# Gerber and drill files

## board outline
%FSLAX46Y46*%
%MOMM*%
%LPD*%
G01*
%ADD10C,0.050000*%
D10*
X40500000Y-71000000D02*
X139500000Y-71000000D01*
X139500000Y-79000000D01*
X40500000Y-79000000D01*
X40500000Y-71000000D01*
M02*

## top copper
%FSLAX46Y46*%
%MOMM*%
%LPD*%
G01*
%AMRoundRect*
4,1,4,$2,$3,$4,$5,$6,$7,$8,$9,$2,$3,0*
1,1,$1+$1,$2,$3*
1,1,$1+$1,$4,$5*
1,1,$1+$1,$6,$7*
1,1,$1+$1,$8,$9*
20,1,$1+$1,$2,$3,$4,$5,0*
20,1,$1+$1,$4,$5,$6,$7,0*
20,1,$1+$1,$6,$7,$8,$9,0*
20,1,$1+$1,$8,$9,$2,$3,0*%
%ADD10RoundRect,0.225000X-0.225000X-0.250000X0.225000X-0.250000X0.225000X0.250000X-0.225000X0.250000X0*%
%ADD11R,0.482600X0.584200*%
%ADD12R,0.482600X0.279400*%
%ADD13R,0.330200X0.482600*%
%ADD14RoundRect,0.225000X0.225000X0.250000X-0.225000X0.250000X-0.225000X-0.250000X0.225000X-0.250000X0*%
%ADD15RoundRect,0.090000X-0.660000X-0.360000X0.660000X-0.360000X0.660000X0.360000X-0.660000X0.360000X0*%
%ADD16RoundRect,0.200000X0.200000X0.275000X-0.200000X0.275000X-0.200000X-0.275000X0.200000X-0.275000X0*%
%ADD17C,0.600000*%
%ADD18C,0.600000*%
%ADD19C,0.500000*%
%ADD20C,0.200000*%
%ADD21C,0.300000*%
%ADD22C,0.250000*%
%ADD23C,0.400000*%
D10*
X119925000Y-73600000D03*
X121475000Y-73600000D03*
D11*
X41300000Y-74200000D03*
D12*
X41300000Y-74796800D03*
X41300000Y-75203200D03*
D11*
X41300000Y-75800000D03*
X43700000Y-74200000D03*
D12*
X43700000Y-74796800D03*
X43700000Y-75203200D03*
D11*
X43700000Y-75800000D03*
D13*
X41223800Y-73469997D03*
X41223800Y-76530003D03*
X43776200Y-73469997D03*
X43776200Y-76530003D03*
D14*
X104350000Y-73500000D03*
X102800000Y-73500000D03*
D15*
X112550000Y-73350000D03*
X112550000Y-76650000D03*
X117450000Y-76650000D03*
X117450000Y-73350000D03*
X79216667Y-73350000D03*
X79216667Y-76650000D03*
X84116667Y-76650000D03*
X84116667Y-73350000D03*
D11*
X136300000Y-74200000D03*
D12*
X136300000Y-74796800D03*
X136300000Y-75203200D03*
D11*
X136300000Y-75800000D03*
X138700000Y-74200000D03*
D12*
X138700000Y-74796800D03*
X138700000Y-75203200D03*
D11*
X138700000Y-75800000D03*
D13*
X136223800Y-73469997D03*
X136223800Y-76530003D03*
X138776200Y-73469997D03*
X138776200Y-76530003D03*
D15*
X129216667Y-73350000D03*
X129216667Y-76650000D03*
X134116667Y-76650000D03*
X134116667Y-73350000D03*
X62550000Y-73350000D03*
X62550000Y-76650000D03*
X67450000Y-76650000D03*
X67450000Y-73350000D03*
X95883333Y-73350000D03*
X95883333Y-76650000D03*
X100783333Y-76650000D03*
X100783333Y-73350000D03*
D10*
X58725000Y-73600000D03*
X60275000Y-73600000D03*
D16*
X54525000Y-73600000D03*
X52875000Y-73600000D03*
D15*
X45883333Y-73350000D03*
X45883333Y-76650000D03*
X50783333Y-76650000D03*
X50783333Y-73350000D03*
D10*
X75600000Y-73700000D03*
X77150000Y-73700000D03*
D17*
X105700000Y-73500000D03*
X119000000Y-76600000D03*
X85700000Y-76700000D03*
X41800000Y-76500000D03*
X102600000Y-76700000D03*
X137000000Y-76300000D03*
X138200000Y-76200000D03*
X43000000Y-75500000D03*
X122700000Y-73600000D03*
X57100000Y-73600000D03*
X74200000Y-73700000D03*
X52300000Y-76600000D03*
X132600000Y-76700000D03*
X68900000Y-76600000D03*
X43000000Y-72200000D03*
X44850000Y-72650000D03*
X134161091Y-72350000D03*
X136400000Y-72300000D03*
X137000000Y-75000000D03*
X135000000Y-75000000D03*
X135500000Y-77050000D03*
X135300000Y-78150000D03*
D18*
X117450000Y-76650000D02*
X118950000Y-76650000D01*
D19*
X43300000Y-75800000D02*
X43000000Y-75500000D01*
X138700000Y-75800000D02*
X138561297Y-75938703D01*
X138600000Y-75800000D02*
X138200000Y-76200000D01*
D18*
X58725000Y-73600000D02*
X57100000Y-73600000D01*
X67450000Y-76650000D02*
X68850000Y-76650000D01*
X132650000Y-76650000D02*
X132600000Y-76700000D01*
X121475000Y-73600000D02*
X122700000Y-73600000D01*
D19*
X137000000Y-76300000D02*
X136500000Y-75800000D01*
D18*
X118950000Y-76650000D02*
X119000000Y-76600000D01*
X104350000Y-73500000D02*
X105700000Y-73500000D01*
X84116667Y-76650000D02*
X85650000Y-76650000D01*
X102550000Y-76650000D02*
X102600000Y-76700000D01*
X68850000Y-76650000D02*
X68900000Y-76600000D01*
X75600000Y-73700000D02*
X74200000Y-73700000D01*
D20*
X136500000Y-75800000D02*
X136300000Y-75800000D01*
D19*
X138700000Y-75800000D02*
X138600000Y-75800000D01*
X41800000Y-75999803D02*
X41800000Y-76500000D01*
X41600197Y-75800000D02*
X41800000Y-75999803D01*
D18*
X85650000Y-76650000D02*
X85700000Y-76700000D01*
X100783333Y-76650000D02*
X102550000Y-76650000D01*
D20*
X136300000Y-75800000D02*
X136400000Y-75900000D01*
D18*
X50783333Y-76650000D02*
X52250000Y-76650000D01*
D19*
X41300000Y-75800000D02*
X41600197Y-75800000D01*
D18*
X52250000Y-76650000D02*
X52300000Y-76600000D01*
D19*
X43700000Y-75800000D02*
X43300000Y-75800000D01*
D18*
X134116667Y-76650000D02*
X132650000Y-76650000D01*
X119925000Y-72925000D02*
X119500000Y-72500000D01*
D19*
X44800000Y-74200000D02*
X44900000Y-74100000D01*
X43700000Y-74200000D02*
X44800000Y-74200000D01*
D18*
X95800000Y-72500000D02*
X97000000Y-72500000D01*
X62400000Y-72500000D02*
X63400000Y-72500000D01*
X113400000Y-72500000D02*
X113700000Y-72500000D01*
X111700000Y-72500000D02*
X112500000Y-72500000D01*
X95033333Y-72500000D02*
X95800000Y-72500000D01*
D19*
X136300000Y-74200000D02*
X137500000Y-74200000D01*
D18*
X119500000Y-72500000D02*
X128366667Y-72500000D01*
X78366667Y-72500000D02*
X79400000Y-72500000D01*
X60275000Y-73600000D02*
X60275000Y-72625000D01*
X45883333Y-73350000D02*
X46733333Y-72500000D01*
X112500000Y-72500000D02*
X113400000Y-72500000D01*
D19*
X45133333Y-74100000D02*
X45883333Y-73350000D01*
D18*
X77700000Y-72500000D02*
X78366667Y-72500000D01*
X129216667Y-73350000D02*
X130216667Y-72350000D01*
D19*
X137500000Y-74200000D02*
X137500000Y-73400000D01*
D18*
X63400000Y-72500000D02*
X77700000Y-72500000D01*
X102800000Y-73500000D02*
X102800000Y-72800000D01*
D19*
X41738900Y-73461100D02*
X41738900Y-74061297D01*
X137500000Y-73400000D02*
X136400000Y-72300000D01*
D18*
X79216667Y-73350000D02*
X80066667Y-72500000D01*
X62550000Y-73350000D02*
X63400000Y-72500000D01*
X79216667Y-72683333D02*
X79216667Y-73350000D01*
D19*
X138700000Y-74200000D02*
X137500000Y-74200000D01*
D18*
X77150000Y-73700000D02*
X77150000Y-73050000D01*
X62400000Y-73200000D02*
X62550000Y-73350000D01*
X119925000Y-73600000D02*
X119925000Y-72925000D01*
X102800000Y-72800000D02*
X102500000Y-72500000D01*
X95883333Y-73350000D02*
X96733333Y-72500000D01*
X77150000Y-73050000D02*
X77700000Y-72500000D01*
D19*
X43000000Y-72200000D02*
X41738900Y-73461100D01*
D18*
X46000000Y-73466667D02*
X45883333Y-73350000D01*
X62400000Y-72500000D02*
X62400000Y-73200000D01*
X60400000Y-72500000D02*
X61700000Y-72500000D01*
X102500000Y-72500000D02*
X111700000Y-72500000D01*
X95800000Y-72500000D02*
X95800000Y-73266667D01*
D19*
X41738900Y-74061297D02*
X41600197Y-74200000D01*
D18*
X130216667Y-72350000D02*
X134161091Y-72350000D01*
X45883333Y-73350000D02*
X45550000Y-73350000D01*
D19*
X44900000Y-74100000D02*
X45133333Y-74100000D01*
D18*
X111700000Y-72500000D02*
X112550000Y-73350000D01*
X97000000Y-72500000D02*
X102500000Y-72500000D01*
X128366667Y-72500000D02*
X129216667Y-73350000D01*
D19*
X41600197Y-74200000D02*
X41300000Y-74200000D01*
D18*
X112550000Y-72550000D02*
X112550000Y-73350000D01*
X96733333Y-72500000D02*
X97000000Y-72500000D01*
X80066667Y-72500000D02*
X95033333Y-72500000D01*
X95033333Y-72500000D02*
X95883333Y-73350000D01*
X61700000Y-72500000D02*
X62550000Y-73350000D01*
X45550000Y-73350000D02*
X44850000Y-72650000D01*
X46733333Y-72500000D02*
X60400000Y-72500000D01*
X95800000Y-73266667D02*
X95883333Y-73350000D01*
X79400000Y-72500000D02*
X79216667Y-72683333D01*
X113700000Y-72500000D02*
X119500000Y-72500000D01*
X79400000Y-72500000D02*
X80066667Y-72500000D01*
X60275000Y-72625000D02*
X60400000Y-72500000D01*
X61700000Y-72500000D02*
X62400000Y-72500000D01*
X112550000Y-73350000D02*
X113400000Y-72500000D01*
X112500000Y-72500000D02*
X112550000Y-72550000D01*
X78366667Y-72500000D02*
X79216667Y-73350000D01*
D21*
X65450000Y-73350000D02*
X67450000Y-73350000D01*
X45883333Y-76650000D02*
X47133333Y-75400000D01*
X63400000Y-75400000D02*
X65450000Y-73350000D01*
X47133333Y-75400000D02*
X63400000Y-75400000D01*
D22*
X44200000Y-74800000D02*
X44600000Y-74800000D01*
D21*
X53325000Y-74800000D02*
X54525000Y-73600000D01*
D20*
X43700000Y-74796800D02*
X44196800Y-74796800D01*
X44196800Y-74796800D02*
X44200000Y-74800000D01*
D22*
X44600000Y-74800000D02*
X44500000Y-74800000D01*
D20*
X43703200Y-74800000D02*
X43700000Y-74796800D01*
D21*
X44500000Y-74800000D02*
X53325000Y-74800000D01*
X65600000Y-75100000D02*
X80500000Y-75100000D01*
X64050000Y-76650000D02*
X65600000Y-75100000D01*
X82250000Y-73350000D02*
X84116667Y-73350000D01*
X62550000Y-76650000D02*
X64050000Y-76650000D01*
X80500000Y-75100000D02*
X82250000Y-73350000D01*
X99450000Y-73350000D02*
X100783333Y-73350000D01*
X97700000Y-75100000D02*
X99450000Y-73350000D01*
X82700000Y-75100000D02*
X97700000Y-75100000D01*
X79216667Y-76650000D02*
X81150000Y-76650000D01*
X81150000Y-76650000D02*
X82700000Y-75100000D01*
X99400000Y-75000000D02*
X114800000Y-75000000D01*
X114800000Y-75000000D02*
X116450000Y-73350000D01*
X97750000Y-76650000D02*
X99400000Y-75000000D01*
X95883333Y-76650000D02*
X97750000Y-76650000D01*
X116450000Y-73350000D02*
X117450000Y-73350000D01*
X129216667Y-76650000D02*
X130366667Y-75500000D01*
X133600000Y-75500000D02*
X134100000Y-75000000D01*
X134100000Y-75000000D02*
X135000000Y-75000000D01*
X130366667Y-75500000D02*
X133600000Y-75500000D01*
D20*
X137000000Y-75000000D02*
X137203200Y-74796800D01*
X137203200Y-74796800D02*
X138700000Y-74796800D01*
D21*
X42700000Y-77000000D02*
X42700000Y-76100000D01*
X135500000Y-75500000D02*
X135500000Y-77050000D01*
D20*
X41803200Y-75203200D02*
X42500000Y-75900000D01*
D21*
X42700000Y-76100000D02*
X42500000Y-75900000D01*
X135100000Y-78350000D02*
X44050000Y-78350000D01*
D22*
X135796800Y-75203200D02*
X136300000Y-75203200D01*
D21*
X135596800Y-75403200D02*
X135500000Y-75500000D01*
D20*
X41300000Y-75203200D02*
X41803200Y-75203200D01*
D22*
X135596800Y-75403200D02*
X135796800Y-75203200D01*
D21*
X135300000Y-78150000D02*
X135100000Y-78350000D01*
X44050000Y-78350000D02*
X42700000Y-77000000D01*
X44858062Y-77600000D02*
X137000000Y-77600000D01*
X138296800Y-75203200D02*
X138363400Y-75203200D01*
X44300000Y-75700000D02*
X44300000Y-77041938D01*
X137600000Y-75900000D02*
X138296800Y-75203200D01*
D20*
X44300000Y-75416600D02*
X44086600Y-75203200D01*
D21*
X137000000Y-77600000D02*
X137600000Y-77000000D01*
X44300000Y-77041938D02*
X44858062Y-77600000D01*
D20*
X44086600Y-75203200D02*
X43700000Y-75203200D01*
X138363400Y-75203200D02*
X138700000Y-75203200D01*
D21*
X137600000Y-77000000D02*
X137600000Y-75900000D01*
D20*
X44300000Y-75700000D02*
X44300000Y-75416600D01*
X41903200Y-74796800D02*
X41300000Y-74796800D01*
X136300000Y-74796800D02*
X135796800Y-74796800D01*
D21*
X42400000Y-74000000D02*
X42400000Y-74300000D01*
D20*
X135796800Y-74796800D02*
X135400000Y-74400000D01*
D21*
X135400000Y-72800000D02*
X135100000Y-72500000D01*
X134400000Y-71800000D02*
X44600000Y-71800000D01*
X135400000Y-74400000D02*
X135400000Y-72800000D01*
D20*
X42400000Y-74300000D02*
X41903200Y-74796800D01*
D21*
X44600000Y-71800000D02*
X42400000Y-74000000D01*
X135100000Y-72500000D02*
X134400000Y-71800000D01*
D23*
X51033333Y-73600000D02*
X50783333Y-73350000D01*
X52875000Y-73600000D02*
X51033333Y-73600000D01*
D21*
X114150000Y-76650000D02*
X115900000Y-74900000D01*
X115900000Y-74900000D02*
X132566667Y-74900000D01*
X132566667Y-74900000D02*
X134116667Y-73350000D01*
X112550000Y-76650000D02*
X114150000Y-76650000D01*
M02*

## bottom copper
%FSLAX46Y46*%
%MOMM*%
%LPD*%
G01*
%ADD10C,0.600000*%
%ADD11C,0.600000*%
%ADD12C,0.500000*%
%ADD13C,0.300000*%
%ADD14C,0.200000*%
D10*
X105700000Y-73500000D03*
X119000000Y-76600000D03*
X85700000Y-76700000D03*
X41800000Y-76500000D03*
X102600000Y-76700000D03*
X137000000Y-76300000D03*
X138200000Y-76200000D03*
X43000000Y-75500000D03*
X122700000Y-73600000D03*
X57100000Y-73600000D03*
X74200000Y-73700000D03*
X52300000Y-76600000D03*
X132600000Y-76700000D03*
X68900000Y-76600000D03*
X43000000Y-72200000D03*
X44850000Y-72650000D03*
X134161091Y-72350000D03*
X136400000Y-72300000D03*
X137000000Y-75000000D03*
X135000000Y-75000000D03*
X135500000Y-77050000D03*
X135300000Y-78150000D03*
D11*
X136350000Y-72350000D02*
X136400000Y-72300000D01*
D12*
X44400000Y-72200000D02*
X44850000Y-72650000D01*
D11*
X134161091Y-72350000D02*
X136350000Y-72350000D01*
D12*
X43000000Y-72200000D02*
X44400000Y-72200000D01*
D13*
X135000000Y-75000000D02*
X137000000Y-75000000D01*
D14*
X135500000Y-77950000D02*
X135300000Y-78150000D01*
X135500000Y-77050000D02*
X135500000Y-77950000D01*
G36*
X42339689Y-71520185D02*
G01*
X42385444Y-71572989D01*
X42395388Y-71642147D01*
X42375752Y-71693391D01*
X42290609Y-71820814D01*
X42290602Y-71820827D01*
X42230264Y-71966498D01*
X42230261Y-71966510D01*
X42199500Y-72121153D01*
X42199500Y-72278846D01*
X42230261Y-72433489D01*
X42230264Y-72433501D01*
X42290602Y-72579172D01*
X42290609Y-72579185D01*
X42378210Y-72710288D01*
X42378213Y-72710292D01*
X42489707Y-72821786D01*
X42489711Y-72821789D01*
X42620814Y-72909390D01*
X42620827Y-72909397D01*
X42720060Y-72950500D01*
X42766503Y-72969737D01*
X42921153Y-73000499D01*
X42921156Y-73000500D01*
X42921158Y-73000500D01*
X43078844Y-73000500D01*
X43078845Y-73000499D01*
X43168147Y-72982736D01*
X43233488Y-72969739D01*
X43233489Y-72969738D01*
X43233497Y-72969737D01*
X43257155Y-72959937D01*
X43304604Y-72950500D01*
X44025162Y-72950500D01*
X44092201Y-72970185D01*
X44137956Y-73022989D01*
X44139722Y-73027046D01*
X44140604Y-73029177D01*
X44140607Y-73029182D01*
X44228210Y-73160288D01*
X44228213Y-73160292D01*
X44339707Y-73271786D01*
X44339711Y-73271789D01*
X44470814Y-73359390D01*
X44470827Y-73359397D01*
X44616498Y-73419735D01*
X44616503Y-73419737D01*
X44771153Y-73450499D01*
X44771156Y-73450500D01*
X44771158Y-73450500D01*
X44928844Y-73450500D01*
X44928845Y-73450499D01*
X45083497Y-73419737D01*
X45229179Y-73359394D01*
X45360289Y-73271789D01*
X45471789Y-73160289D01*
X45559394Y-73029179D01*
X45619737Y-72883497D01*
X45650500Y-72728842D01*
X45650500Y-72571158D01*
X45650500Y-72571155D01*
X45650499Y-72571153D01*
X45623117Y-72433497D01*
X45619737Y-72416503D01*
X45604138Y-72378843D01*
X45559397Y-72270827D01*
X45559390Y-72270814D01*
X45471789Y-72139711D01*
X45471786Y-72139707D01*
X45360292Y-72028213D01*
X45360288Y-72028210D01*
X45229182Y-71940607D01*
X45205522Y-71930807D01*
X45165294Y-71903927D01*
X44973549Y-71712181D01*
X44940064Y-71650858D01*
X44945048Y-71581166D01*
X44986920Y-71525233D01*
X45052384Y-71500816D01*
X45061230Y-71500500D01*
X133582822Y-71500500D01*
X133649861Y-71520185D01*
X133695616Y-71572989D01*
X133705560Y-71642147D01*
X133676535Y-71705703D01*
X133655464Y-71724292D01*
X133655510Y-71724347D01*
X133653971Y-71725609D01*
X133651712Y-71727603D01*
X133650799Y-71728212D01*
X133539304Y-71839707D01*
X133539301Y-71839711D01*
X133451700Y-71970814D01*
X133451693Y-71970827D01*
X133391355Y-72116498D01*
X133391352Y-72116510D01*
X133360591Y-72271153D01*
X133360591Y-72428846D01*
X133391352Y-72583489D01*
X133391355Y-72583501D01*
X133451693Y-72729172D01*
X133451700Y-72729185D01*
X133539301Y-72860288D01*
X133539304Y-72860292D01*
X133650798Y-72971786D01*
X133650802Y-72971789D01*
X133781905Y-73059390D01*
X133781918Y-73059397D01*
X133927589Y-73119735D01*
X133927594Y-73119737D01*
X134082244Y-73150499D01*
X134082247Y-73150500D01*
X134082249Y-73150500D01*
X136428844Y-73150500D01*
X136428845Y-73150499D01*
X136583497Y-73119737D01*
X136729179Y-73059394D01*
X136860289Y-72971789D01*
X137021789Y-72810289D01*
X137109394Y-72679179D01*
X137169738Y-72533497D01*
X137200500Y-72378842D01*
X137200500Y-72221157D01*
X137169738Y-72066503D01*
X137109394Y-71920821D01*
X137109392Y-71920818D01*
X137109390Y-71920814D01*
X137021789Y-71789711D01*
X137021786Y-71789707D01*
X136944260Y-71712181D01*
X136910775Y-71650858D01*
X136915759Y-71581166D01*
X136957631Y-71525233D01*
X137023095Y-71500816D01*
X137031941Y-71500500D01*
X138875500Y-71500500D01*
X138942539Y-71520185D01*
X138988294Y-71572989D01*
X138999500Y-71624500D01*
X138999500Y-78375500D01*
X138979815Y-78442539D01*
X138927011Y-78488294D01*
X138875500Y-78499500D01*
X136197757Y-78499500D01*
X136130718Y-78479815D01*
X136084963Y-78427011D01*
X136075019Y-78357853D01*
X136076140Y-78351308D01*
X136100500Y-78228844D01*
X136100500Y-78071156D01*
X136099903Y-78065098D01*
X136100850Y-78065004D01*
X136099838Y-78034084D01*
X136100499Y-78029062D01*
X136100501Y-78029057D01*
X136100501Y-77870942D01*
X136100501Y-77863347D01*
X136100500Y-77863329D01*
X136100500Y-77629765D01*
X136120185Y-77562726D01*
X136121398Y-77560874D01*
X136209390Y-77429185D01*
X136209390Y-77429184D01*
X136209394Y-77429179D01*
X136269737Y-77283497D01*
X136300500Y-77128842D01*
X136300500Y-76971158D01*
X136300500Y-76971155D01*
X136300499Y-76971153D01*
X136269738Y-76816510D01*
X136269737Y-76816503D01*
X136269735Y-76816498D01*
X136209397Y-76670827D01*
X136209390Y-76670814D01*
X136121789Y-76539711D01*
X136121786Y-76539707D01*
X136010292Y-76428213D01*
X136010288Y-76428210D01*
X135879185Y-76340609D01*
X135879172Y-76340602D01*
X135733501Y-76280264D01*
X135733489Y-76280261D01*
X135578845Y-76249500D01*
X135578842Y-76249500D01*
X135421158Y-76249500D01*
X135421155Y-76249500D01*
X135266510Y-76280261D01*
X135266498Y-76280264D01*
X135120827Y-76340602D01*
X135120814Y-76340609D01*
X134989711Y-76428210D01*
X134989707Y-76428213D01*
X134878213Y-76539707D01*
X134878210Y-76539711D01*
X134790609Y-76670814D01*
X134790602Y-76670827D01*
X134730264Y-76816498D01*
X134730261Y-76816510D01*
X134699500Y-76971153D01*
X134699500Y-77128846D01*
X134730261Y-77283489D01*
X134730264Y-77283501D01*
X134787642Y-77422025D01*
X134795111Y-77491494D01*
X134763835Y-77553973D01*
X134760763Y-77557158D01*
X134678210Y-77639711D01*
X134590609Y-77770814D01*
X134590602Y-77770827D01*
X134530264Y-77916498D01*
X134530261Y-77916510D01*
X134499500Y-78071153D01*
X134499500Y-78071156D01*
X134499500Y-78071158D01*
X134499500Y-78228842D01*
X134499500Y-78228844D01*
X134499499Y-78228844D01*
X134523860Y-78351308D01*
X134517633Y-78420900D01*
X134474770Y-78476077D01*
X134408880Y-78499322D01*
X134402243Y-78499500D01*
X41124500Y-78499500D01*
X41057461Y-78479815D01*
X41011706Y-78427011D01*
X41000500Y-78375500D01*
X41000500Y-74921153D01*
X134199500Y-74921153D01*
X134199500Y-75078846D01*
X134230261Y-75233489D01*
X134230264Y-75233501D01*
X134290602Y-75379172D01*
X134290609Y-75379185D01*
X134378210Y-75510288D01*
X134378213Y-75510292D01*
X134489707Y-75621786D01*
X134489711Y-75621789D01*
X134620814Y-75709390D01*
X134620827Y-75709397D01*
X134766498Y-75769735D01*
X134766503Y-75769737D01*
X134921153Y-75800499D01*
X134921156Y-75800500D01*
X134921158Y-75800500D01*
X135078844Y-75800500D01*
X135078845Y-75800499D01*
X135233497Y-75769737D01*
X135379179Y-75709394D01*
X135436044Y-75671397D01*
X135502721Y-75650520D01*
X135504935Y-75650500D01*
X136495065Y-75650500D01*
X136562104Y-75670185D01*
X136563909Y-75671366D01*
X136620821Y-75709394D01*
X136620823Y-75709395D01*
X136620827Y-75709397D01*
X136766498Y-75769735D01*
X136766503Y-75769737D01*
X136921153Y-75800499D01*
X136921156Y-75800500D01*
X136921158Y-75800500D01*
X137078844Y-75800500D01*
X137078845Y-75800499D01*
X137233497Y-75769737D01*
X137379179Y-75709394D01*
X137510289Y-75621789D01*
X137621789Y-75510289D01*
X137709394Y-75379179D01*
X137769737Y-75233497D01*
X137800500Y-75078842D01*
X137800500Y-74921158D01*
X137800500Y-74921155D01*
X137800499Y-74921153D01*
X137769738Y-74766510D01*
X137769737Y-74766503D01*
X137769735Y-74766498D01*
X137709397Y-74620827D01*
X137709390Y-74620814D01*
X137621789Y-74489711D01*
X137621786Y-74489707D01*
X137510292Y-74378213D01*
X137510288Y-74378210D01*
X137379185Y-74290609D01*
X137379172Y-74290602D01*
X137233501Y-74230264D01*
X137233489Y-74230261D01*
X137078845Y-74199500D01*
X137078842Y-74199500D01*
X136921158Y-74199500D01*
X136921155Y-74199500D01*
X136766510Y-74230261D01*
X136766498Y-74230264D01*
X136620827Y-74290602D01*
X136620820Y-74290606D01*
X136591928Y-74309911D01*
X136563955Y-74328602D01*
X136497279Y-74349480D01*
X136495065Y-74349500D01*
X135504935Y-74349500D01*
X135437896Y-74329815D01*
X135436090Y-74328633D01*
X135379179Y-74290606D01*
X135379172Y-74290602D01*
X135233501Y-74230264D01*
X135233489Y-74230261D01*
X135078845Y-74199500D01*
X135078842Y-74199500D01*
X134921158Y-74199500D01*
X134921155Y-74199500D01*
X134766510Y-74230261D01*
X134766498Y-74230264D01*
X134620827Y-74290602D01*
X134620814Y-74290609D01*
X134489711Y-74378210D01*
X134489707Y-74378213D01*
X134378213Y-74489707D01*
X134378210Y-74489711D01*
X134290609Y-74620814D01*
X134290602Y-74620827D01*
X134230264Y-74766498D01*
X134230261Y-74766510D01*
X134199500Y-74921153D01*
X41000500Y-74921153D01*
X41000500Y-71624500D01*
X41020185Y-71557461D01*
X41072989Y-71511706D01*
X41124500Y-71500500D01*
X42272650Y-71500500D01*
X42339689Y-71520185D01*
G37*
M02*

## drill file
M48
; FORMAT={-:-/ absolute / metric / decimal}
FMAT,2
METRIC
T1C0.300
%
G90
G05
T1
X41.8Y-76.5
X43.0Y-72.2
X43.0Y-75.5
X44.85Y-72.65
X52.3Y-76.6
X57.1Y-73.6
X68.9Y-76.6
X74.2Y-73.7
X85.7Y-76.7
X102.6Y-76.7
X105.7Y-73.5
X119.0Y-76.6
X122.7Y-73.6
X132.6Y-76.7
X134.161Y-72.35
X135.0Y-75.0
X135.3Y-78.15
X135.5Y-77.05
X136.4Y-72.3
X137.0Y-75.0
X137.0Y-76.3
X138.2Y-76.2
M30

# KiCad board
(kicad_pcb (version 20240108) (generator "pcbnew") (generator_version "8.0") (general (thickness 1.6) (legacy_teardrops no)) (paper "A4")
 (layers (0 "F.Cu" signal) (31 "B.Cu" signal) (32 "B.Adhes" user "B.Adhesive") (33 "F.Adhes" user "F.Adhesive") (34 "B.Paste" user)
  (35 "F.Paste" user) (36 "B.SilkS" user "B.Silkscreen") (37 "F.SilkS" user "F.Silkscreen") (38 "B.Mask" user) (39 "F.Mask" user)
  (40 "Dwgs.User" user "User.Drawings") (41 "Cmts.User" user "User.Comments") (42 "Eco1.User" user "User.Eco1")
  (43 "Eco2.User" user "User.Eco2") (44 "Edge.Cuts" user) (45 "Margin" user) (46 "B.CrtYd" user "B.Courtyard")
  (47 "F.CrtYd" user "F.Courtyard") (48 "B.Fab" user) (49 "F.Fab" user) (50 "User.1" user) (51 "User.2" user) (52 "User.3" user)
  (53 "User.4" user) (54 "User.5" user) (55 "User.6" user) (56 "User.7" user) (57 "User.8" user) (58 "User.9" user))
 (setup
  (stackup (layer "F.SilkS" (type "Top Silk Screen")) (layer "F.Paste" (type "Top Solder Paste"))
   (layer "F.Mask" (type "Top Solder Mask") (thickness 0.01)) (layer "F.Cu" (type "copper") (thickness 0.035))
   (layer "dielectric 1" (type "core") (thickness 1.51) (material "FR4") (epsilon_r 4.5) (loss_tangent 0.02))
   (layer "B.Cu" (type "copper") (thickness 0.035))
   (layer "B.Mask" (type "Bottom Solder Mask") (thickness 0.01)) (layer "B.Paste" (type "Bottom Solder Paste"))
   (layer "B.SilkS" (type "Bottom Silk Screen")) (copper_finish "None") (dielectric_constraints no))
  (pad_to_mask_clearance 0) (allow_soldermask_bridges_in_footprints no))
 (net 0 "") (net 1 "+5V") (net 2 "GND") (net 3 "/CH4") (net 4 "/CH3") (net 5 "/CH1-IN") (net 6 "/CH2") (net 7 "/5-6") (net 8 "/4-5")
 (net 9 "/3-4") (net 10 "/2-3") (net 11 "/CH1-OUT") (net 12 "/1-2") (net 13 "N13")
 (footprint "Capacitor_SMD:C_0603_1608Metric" (layer "F.Cu") (at 120.7 73.6)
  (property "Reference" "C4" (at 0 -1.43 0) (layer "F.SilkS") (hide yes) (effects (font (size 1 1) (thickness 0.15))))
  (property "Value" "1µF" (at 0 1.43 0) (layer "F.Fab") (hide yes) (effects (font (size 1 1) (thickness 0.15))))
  (pad "1" smd roundrect (at -0.775 0) (size 0.9 0.95) (layers "F.Cu" "F.Paste" "F.Mask") (roundrect_rratio 0.25) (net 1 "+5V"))
  (pad "2" smd roundrect (at 0.775 0) (size 0.9 0.95) (layers "F.Cu" "F.Paste" "F.Mask") (roundrect_rratio 0.25) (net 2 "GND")))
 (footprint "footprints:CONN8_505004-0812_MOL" (layer "F.Cu") (at 42.5 75 90)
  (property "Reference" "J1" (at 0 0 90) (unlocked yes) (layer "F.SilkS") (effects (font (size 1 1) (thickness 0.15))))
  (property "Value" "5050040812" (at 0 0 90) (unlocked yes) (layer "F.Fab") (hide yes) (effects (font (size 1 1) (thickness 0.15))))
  (pad "1" smd rect (at 0.8 -1.2 90) (size 0.5842 0.4826) (layers "F.Cu" "F.Paste" "F.Mask") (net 1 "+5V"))
  (pad "2" smd rect (at 0.2032 -1.2 90) (size 0.2794 0.4826) (layers "F.Cu" "F.Paste" "F.Mask") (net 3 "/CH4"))
  (pad "3" smd rect (at -0.2032 -1.2 90) (size 0.2794 0.4826) (layers "F.Cu" "F.Paste" "F.Mask") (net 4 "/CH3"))
  (pad "4" smd rect (at -0.8 -1.2 90) (size 0.5842 0.4826) (layers "F.Cu" "F.Paste" "F.Mask") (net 2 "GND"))
  (pad "5" smd rect (at 0.8 1.2 90) (size 0.5842 0.4826) (layers "F.Cu" "F.Paste" "F.Mask") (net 1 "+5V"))
  (pad "6" smd rect (at 0.2032 1.2 90) (size 0.2794 0.4826) (layers "F.Cu" "F.Paste" "F.Mask") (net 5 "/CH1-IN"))
  (pad "7" smd rect (at -0.2032 1.2 90) (size 0.2794 0.4826) (layers "F.Cu" "F.Paste" "F.Mask") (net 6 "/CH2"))
  (pad "8" smd rect (at -0.8 1.2 90) (size 0.5842 0.4826) (layers "F.Cu" "F.Paste" "F.Mask") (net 2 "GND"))
  (pad "9" smd rect (at 1.530003 -1.2762 90) (size 0.4826 0.3302) (layers "F.Cu" "F.Paste" "F.Mask"))
  (pad "10" smd rect (at -1.530003 -1.2762 90) (size 0.4826 0.3302) (layers "F.Cu" "F.Paste" "F.Mask"))
  (pad "11" smd rect (at 1.530003 1.2762 90) (size 0.4826 0.3302) (layers "F.Cu" "F.Paste" "F.Mask"))
  (pad "12" smd rect (at -1.530003 1.2762 90) (size 0.4826 0.3302) (layers "F.Cu" "F.Paste" "F.Mask")))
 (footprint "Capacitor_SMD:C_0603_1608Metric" (layer "F.Cu") (at 103.575 73.5 180)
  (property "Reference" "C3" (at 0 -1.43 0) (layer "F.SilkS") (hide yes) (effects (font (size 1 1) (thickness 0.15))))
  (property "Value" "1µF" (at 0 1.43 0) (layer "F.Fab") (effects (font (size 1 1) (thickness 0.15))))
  (pad "1" smd roundrect (at -0.775 0 180) (size 0.9 0.95) (layers "F.Cu" "F.Paste" "F.Mask") (roundrect_rratio 0.25) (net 2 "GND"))
  (pad "2" smd roundrect (at 0.775 0 180) (size 0.9 0.95) (layers "F.Cu" "F.Paste" "F.Mask") (roundrect_rratio 0.25) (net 1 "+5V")))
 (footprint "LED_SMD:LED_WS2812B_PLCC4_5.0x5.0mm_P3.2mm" (layer "F.Cu") (at 115 75)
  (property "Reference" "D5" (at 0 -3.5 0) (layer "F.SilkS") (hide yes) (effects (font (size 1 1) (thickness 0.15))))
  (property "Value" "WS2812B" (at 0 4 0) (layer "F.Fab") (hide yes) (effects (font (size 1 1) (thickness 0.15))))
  (pad "1" smd roundrect (at -2.45 -1.65) (size 1.5 0.9) (layers "F.Cu" "F.Paste" "F.Mask") (roundrect_rratio 0.1) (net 1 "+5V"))
  (pad "2" smd roundrect (at -2.45 1.65) (size 1.5 0.9) (layers "F.Cu" "F.Paste" "F.Mask") (roundrect_rratio 0.1) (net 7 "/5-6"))
  (pad "3" smd roundrect (at 2.45 1.65) (size 1.5 0.9) (layers "F.Cu" "F.Paste" "F.Mask") (roundrect_rratio 0.1) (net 2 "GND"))
  (pad "4" smd roundrect (at 2.45 -1.65) (size 1.5 0.9) (layers "F.Cu" "F.Paste" "F.Mask") (roundrect_rratio 0.1) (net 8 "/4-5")))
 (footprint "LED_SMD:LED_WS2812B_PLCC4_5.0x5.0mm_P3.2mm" (layer "F.Cu") (at 81.666667 75)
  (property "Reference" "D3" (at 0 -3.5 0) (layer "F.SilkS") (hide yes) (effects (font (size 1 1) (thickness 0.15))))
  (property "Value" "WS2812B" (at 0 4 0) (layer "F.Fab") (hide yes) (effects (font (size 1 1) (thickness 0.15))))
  (pad "1" smd roundrect (at -2.45 -1.65) (size 1.5 0.9) (layers "F.Cu" "F.Paste" "F.Mask") (roundrect_rratio 0.1) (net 1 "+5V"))
  (pad "2" smd roundrect (at -2.45 1.65) (size 1.5 0.9) (layers "F.Cu" "F.Paste" "F.Mask") (roundrect_rratio 0.1) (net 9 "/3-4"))
  (pad "3" smd roundrect (at 2.45 1.65) (size 1.5 0.9) (layers "F.Cu" "F.Paste" "F.Mask") (roundrect_rratio 0.1) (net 2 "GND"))
  (pad "4" smd roundrect (at 2.45 -1.65) (size 1.5 0.9) (layers "F.Cu" "F.Paste" "F.Mask") (roundrect_rratio 0.1) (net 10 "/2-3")))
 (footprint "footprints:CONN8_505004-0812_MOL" (layer "F.Cu") (at 137.5 75 90)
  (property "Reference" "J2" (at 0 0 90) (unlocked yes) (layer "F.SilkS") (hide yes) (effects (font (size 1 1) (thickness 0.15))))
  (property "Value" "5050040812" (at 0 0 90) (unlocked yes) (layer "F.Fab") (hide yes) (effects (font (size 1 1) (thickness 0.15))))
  (pad "1" smd rect (at 0.8 -1.2 90) (size 0.5842 0.4826) (layers "F.Cu" "F.Paste" "F.Mask") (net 1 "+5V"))
  (pad "2" smd rect (at 0.2032 -1.2 90) (size 0.2794 0.4826) (layers "F.Cu" "F.Paste" "F.Mask") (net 3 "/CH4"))
  (pad "3" smd rect (at -0.2032 -1.2 90) (size 0.2794 0.4826) (layers "F.Cu" "F.Paste" "F.Mask") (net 4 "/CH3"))
  (pad "4" smd rect (at -0.8 -1.2 90) (size 0.5842 0.4826) (layers "F.Cu" "F.Paste" "F.Mask") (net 2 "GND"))
  (pad "5" smd rect (at 0.8 1.2 90) (size 0.5842 0.4826) (layers "F.Cu" "F.Paste" "F.Mask") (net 1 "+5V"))
  (pad "6" smd rect (at 0.2032 1.2 90) (size 0.2794 0.4826) (layers "F.Cu" "F.Paste" "F.Mask") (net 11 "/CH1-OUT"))
  (pad "7" smd rect (at -0.2032 1.2 90) (size 0.2794 0.4826) (layers "F.Cu" "F.Paste" "F.Mask") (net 6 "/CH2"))
  (pad "8" smd rect (at -0.8 1.2 90) (size 0.5842 0.4826) (layers "F.Cu" "F.Paste" "F.Mask") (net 2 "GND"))
  (pad "9" smd rect (at 1.530003 -1.2762 90) (size 0.4826 0.3302) (layers "F.Cu" "F.Paste" "F.Mask"))
  (pad "10" smd rect (at -1.530003 -1.2762 90) (size 0.4826 0.3302) (layers "F.Cu" "F.Paste" "F.Mask"))
  (pad "11" smd rect (at 1.530003 1.2762 90) (size 0.4826 0.3302) (layers "F.Cu" "F.Paste" "F.Mask"))
  (pad "12" smd rect (at -1.530003 1.2762 90) (size 0.4826 0.3302) (layers "F.Cu" "F.Paste" "F.Mask")))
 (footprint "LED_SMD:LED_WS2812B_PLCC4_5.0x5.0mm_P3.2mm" (layer "F.Cu") (at 131.666667 75)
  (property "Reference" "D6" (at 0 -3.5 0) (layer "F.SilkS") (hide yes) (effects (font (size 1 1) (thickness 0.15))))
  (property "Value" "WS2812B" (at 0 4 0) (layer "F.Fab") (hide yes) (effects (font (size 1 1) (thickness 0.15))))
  (pad "1" smd roundrect (at -2.45 -1.65) (size 1.5 0.9) (layers "F.Cu" "F.Paste" "F.Mask") (roundrect_rratio 0.1) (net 1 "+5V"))
  (pad "2" smd roundrect (at -2.45 1.65) (size 1.5 0.9) (layers "F.Cu" "F.Paste" "F.Mask") (roundrect_rratio 0.1) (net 11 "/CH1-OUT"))
  (pad "3" smd roundrect (at 2.45 1.65) (size 1.5 0.9) (layers "F.Cu" "F.Paste" "F.Mask") (roundrect_rratio 0.1) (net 2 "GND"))
  (pad "4" smd roundrect (at 2.45 -1.65) (size 1.5 0.9) (layers "F.Cu" "F.Paste" "F.Mask") (roundrect_rratio 0.1) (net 7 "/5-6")))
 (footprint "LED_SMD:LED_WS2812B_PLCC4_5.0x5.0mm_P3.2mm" (layer "F.Cu") (at 65 75)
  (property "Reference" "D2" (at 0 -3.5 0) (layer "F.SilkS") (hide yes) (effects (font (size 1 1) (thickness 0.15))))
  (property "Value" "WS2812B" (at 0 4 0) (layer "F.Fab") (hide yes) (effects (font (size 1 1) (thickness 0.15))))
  (pad "1" smd roundrect (at -2.45 -1.65) (size 1.5 0.9) (layers "F.Cu" "F.Paste" "F.Mask") (roundrect_rratio 0.1) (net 1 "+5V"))
  (pad "2" smd roundrect (at -2.45 1.65) (size 1.5 0.9) (layers "F.Cu" "F.Paste" "F.Mask") (roundrect_rratio 0.1) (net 10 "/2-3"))
  (pad "3" smd roundrect (at 2.45 1.65) (size 1.5 0.9) (layers "F.Cu" "F.Paste" "F.Mask") (roundrect_rratio 0.1) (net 2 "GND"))
  (pad "4" smd roundrect (at 2.45 -1.65) (size 1.5 0.9) (layers "F.Cu" "F.Paste" "F.Mask") (roundrect_rratio 0.1) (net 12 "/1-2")))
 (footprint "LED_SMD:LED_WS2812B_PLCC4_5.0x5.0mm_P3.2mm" (layer "F.Cu") (at 98.333333 75)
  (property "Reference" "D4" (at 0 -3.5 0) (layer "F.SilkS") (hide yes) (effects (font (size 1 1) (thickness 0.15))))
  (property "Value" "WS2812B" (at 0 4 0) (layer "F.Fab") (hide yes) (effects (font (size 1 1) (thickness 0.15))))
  (pad "1" smd roundrect (at -2.45 -1.65) (size 1.5 0.9) (layers "F.Cu" "F.Paste" "F.Mask") (roundrect_rratio 0.1) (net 1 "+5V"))
  (pad "2" smd roundrect (at -2.45 1.65) (size 1.5 0.9) (layers "F.Cu" "F.Paste" "F.Mask") (roundrect_rratio 0.1) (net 8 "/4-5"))
  (pad "3" smd roundrect (at 2.45 1.65) (size 1.5 0.9) (layers "F.Cu" "F.Paste" "F.Mask") (roundrect_rratio 0.1) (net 2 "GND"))
  (pad "4" smd roundrect (at 2.45 -1.65) (size 1.5 0.9) (layers "F.Cu" "F.Paste" "F.Mask") (roundrect_rratio 0.1) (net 9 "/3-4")))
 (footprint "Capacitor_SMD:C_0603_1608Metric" (layer "F.Cu") (at 59.5 73.6)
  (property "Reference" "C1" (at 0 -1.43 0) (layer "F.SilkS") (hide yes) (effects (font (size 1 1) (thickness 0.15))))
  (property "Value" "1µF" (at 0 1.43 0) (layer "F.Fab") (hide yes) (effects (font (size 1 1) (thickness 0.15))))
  (pad "1" smd roundrect (at -0.775 0) (size 0.9 0.95) (layers "F.Cu" "F.Paste" "F.Mask") (roundrect_rratio 0.25) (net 2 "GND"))
  (pad "2" smd roundrect (at 0.775 0) (size 0.9 0.95) (layers "F.Cu" "F.Paste" "F.Mask") (roundrect_rratio 0.25) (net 1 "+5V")))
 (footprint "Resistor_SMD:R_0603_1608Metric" (layer "F.Cu") (at 53.7 73.6 180)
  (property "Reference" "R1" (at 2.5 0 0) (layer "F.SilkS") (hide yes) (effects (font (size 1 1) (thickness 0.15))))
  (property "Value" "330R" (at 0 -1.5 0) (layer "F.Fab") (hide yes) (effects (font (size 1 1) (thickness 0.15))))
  (pad "1" smd roundrect (at -0.825 0 180) (size 0.8 0.95) (layers "F.Cu" "F.Paste" "F.Mask") (roundrect_rratio 0.25) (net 5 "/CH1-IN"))
  (pad "2" smd roundrect (at 0.825 0 180) (size 0.8 0.95) (layers "F.Cu" "F.Paste" "F.Mask") (roundrect_rratio 0.25) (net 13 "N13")))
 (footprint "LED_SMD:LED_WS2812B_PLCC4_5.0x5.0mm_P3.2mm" (layer "F.Cu") (at 48.333333 75)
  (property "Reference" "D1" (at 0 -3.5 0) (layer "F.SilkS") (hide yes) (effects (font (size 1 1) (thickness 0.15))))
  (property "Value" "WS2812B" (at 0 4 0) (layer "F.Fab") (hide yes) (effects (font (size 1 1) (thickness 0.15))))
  (pad "1" smd roundrect (at -2.45 -1.65) (size 1.5 0.9) (layers "F.Cu" "F.Paste" "F.Mask") (roundrect_rratio 0.1) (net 1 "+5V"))
  (pad "2" smd roundrect (at -2.45 1.65) (size 1.5 0.9) (layers "F.Cu" "F.Paste" "F.Mask") (roundrect_rratio 0.1) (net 12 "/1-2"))
  (pad "3" smd roundrect (at 2.45 1.65) (size 1.5 0.9) (layers "F.Cu" "F.Paste" "F.Mask") (roundrect_rratio 0.1) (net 2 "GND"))
  (pad "4" smd roundrect (at 2.45 -1.65) (size 1.5 0.9) (layers "F.Cu" "F.Paste" "F.Mask") (roundrect_rratio 0.1) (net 13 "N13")))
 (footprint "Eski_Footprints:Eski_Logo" (layer "F.Cu") (at 90 76.85)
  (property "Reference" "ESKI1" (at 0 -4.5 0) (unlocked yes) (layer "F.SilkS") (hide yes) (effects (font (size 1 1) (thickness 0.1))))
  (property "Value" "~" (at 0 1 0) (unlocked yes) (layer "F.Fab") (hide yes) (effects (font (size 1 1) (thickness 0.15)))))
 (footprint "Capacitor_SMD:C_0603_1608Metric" (layer "F.Cu") (at 76.375 73.7)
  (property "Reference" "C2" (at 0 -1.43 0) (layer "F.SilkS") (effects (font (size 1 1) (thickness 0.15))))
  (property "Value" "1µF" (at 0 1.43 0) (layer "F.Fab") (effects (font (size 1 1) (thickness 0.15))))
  (pad "1" smd roundrect (at -0.775 0) (size 0.9 0.95) (layers "F.Cu" "F.Paste" "F.Mask") (roundrect_rratio 0.25) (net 2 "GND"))
  (pad "2" smd roundrect (at 0.775 0) (size 0.9 0.95) (layers "F.Cu" "F.Paste" "F.Mask") (roundrect_rratio 0.25) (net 1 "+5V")))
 (gr_rect (start 40.5 71) (end 139.5 79) (stroke (width 0.05) (type default)) (fill none) (layer "Edge.Cuts"))
 (segment (start 117.45 76.65) (end 118.95 76.65) (width 0.6) (layer "F.Cu") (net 2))
 (segment (start 43.3 75.8) (end 43 75.5) (width 0.5) (layer "F.Cu") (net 2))
 (segment (start 138.7 75.8) (end 138.561297 75.938703) (width 0.5) (layer "F.Cu") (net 2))
 (segment (start 138.6 75.8) (end 138.2 76.2) (width 0.5) (layer "F.Cu") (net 2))
 (segment (start 58.725 73.6) (end 57.1 73.6) (width 0.6) (layer "F.Cu") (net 2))
 (segment (start 67.45 76.65) (end 68.85 76.65) (width 0.6) (layer "F.Cu") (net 2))
 (segment (start 132.65 76.65) (end 132.6 76.7) (width 0.6) (layer "F.Cu") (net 2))
 (segment (start 121.475 73.6) (end 122.7 73.6) (width 0.6) (layer "F.Cu") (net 2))
 (segment (start 137 76.3) (end 136.5 75.8) (width 0.5) (layer "F.Cu") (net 2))
 (segment (start 118.95 76.65) (end 119 76.6) (width 0.6) (layer "F.Cu") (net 2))
 (segment (start 104.35 73.5) (end 105.7 73.5) (width 0.6) (layer "F.Cu") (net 2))
 (segment (start 84.116667 76.65) (end 85.65 76.65) (width 0.6) (layer "F.Cu") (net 2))
 (segment (start 102.55 76.65) (end 102.6 76.7) (width 0.6) (layer "F.Cu") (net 2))
 (segment (start 68.85 76.65) (end 68.9 76.6) (width 0.6) (layer "F.Cu") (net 2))
 (segment (start 75.6 73.7) (end 74.2 73.7) (width 0.6) (layer "F.Cu") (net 2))
 (segment (start 136.5 75.8) (end 136.3 75.8) (width 0.2) (layer "F.Cu") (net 2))
 (segment (start 138.7 75.8) (end 138.6 75.8) (width 0.5) (layer "F.Cu") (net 2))
 (segment (start 41.8 75.999803) (end 41.8 76.5) (width 0.5) (layer "F.Cu") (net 2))
 (segment (start 41.600197 75.8) (end 41.8 75.999803) (width 0.5) (layer "F.Cu") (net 2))
 (segment (start 85.65 76.65) (end 85.7 76.7) (width 0.6) (layer "F.Cu") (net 2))
 (segment (start 100.783333 76.65) (end 102.55 76.65) (width 0.6) (layer "F.Cu") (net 2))
 (segment (start 136.3 75.8) (end 136.4 75.9) (width 0.2) (layer "F.Cu") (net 2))
 (segment (start 50.783333 76.65) (end 52.25 76.65) (width 0.6) (layer "F.Cu") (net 2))
 (segment (start 41.3 75.8) (end 41.600197 75.8) (width 0.5) (layer "F.Cu") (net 2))
 (segment (start 52.25 76.65) (end 52.3 76.6) (width 0.6) (layer "F.Cu") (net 2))
 (segment (start 43.7 75.8) (end 43.3 75.8) (width 0.5) (layer "F.Cu") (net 2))
 (segment (start 134.116667 76.65) (end 132.65 76.65) (width 0.6) (layer "F.Cu") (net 2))
 (via (at 105.7 73.5) (size 0.6) (drill 0.3) (layers "F.Cu" "B.Cu") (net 2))
 (via (at 119 76.6) (size 0.6) (drill 0.3) (layers "F.Cu" "B.Cu") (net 2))
 (via (at 85.7 76.7) (size 0.6) (drill 0.3) (layers "F.Cu" "B.Cu") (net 2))
 (via (at 41.8 76.5) (size 0.6) (drill 0.3) (layers "F.Cu" "B.Cu") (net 2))
 (via (at 102.6 76.7) (size 0.6) (drill 0.3) (layers "F.Cu" "B.Cu") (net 2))
 (via (at 137 76.3) (size 0.6) (drill 0.3) (layers "F.Cu" "B.Cu") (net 2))
 (via (at 138.2 76.2) (size 0.6) (drill 0.3) (layers "F.Cu" "B.Cu") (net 2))
 (via (at 43 75.5) (size 0.6) (drill 0.3) (layers "F.Cu" "B.Cu") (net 2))
 (via (at 122.7 73.6) (size 0.6) (drill 0.3) (layers "F.Cu" "B.Cu") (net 2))
 (via (at 57.1 73.6) (size 0.6) (drill 0.3) (layers "F.Cu" "B.Cu") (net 2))
 (via (at 74.2 73.7) (size 0.6) (drill 0.3) (layers "F.Cu" "B.Cu") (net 2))
 (via (at 52.3 76.6) (size 0.6) (drill 0.3) (layers "F.Cu" "B.Cu") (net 2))
 (via (at 132.6 76.7) (size 0.6) (drill 0.3) (layers "F.Cu" "B.Cu") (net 2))
 (via (at 68.9 76.6) (size 0.6) (drill 0.3) (layers "F.Cu" "B.Cu") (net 2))
 (segment (start 119.925 72.925) (end 119.5 72.5) (width 0.6) (layer "F.Cu") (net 1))
 (segment (start 44.8 74.2) (end 44.9 74.1) (width 0.5) (layer "F.Cu") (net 1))
 (segment (start 43.7 74.2) (end 44.8 74.2) (width 0.5) (layer "F.Cu") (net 1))
 (segment (start 95.8 72.5) (end 97 72.5) (width 0.6) (layer "F.Cu") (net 1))
 (segment (start 62.4 72.5) (end 63.4 72.5) (width 0.6) (layer "F.Cu") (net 1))
 (segment (start 113.4 72.5) (end 113.7 72.5) (width 0.6) (layer "F.Cu") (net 1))
 (segment (start 111.7 72.5) (end 112.5 72.5) (width 0.6) (layer "F.Cu") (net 1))
 (segment (start 95.033333 72.5) (end 95.8 72.5) (width 0.6) (layer "F.Cu") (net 1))
 (segment (start 136.3 74.2) (end 137.5 74.2) (width 0.5) (layer "F.Cu") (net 1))
 (segment (start 119.5 72.5) (end 128.366667 72.5) (width 0.6) (layer "F.Cu") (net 1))
 (segment (start 78.366667 72.5) (end 79.4 72.5) (width 0.6) (layer "F.Cu") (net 1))
 (segment (start 60.275 73.6) (end 60.275 72.625) (width 0.6) (layer "F.Cu") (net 1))
 (segment (start 45.883333 73.35) (end 46.733333 72.5) (width 0.6) (layer "F.Cu") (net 1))
 (segment (start 112.5 72.5) (end 113.4 72.5) (width 0.6) (layer "F.Cu") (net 1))
 (segment (start 45.133333 74.1) (end 45.883333 73.35) (width 0.5) (layer "F.Cu") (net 1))
 (segment (start 77.7 72.5) (end 78.366667 72.5) (width 0.6) (layer "F.Cu") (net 1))
 (segment (start 129.216667 73.35) (end 130.216667 72.35) (width 0.6) (layer "F.Cu") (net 1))
 (segment (start 137.5 74.2) (end 137.5 73.4) (width 0.5) (layer "F.Cu") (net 1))
 (segment (start 63.4 72.5) (end 77.7 72.5) (width 0.6) (layer "F.Cu") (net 1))
 (segment (start 102.8 73.5) (end 102.8 72.8) (width 0.6) (layer "F.Cu") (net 1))
 (segment (start 41.7389 73.4611) (end 41.7389 74.061297) (width 0.5) (layer "F.Cu") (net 1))
 (segment (start 137.5 73.4) (end 136.4 72.3) (width 0.5) (layer "F.Cu") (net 1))
 (segment (start 79.216667 73.35) (end 80.066667 72.5) (width 0.6) (layer "F.Cu") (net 1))
 (segment (start 62.55 73.35) (end 63.4 72.5) (width 0.6) (layer "F.Cu") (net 1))
 (segment (start 79.216667 72.683333) (end 79.216667 73.35) (width 0.6) (layer "F.Cu") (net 1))
 (segment (start 138.7 74.2) (end 137.5 74.2) (width 0.5) (layer "F.Cu") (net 1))
 (segment (start 77.15 73.7) (end 77.15 73.05) (width 0.6) (layer "F.Cu") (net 1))
 (segment (start 62.4 73.2) (end 62.55 73.35) (width 0.6) (layer "F.Cu") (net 1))
 (segment (start 119.925 73.6) (end 119.925 72.925) (width 0.6) (layer "F.Cu") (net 1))
 (segment (start 102.8 72.8) (end 102.5 72.5) (width 0.6) (layer "F.Cu") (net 1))
 (segment (start 95.883333 73.35) (end 96.733333 72.5) (width 0.6) (layer "F.Cu") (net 1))
 (segment (start 77.15 73.05) (end 77.7 72.5) (width 0.6) (layer "F.Cu") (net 1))
 (segment (start 43 72.2) (end 41.7389 73.4611) (width 0.5) (layer "F.Cu") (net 1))
 (segment (start 46 73.466667) (end 45.883333 73.35) (width 0.6) (layer "F.Cu") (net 1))
 (segment (start 62.4 72.5) (end 62.4 73.2) (width 0.6) (layer "F.Cu") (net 1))
 (segment (start 60.4 72.5) (end 61.7 72.5) (width 0.6) (layer "F.Cu") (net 1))
 (segment (start 102.5 72.5) (end 111.7 72.5) (width 0.6) (layer "F.Cu") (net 1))
 (segment (start 95.8 72.5) (end 95.8 73.266667) (width 0.6) (layer "F.Cu") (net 1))
 (segment (start 41.7389 74.061297) (end 41.600197 74.2) (width 0.5) (layer "F.Cu") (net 1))
 (segment (start 130.216667 72.35) (end 134.161091 72.35) (width 0.6) (layer "F.Cu") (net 1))
 (segment (start 45.883333 73.35) (end 45.55 73.35) (width 0.6) (layer "F.Cu") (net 1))
 (segment (start 44.9 74.1) (end 45.133333 74.1) (width 0.5) (layer "F.Cu") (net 1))
 (segment (start 111.7 72.5) (end 112.55 73.35) (width 0.6) (layer "F.Cu") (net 1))
 (segment (start 97 72.5) (end 102.5 72.5) (width 0.6) (layer "F.Cu") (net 1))
 (segment (start 128.366667 72.5) (end 129.216667 73.35) (width 0.6) (layer "F.Cu") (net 1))
 (segment (start 41.600197 74.2) (end 41.3 74.2) (width 0.5) (layer "F.Cu") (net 1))
 (segment (start 112.55 72.55) (end 112.55 73.35) (width 0.6) (layer "F.Cu") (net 1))
 (segment (start 96.733333 72.5) (end 97 72.5) (width 0.6) (layer "F.Cu") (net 1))
 (segment (start 80.066667 72.5) (end 95.033333 72.5) (width 0.6) (layer "F.Cu") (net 1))
 (segment (start 95.033333 72.5) (end 95.883333 73.35) (width 0.6) (layer "F.Cu") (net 1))
 (segment (start 61.7 72.5) (end 62.55 73.35) (width 0.6) (layer "F.Cu") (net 1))
 (segment (start 45.55 73.35) (end 44.85 72.65) (width 0.6) (layer "F.Cu") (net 1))
 (segment (start 46.733333 72.5) (end 60.4 72.5) (width 0.6) (layer "F.Cu") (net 1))
 (segment (start 95.8 73.266667) (end 95.883333 73.35) (width 0.6) (layer "F.Cu") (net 1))
 (segment (start 79.4 72.5) (end 79.216667 72.683333) (width 0.6) (layer "F.Cu") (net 1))
 (segment (start 113.7 72.5) (end 119.5 72.5) (width 0.6) (layer "F.Cu") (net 1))
 (segment (start 79.4 72.5) (end 80.066667 72.5) (width 0.6) (layer "F.Cu") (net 1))
 (segment (start 60.275 72.625) (end 60.4 72.5) (width 0.6) (layer "F.Cu") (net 1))
 (segment (start 61.7 72.5) (end 62.4 72.5) (width 0.6) (layer "F.Cu") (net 1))
 (segment (start 112.55 73.35) (end 113.4 72.5) (width 0.6) (layer "F.Cu") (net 1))
 (segment (start 112.5 72.5) (end 112.55 72.55) (width 0.6) (layer "F.Cu") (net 1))
 (segment (start 78.366667 72.5) (end 79.216667 73.35) (width 0.6) (layer "F.Cu") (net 1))
 (via (at 43 72.2) (size 0.6) (drill 0.3) (layers "F.Cu" "B.Cu") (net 1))
 (via (at 44.85 72.65) (size 0.6) (drill 0.3) (layers "F.Cu" "B.Cu") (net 1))
 (via (at 134.161091 72.35) (size 0.6) (drill 0.3) (layers "F.Cu" "B.Cu") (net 1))
 (via (at 136.4 72.3) (size 0.6) (drill 0.3) (layers "F.Cu" "B.Cu") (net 1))
 (segment (start 136.35 72.35) (end 136.4 72.3) (width 0.6) (layer "B.Cu") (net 1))
 (segment (start 44.4 72.2) (end 44.85 72.65) (width 0.5) (layer "B.Cu") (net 1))
 (segment (start 134.161091 72.35) (end 136.35 72.35) (width 0.6) (layer "B.Cu") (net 1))
 (segment (start 43 72.2) (end 44.4 72.2) (width 0.5) (layer "B.Cu") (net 1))
 (segment (start 65.45 73.35) (end 67.45 73.35) (width 0.3) (layer "F.Cu") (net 12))
 (segment (start 45.883333 76.65) (end 47.133333 75.4) (width 0.3) (layer "F.Cu") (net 12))
 (segment (start 63.4 75.4) (end 65.45 73.35) (width 0.3) (layer "F.Cu") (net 12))
 (segment (start 47.133333 75.4) (end 63.4 75.4) (width 0.3) (layer "F.Cu") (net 12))
 (segment (start 44.2 74.8) (end 44.6 74.8) (width 0.25) (layer "F.Cu") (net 5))
 (segment (start 53.325 74.8) (end 54.525 73.6) (width 0.3) (layer "F.Cu") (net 5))
 (segment (start 43.7 74.7968) (end 44.1968 74.7968) (width 0.2) (layer "F.Cu") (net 5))
 (segment (start 44.1968 74.7968) (end 44.2 74.8) (width 0.2) (layer "F.Cu") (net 5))
 (segment (start 44.6 74.8) (end 44.5 74.8) (width 0.25) (layer "F.Cu") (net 5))
 (segment (start 43.7032 74.8) (end 43.7 74.7968) (width 0.2) (layer "F.Cu") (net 5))
 (segment (start 44.5 74.8) (end 53.325 74.8) (width 0.3) (layer "F.Cu") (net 5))
 (segment (start 65.6 75.1) (end 80.5 75.1) (width 0.3) (layer "F.Cu") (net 10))
 (segment (start 64.05 76.65) (end 65.6 75.1) (width 0.3) (layer "F.Cu") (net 10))
 (segment (start 82.25 73.35) (end 84.116667 73.35) (width 0.3) (layer "F.Cu") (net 10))
 (segment (start 62.55 76.65) (end 64.05 76.65) (width 0.3) (layer "F.Cu") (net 10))
 (segment (start 80.5 75.1) (end 82.25 73.35) (width 0.3) (layer "F.Cu") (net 10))
 (segment (start 99.45 73.35) (end 100.783333 73.35) (width 0.3) (layer "F.Cu") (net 9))
 (segment (start 97.7 75.1) (end 99.45 73.35) (width 0.3) (layer "F.Cu") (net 9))
 (segment (start 82.7 75.1) (end 97.7 75.1) (width 0.3) (layer "F.Cu") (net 9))
 (segment (start 79.216667 76.65) (end 81.15 76.65) (width 0.3) (layer "F.Cu") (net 9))
 (segment (start 81.15 76.65) (end 82.7 75.1) (width 0.3) (layer "F.Cu") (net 9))
 (segment (start 99.4 75) (end 114.8 75) (width 0.3) (layer "F.Cu") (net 8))
 (segment (start 114.8 75) (end 116.45 73.35) (width 0.3) (layer "F.Cu") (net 8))
 (segment (start 97.75 76.65) (end 99.4 75) (width 0.3) (layer "F.Cu") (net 8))
 (segment (start 95.883333 76.65) (end 97.75 76.65) (width 0.3) (layer "F.Cu") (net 8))
 (segment (start 116.45 73.35) (end 117.45 73.35) (width 0.3) (layer "F.Cu") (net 8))
 (segment (start 129.216667 76.65) (end 130.366667 75.5) (width 0.3) (layer "F.Cu") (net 11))
 (segment (start 133.6 75.5) (end 134.1 75) (width 0.3) (layer "F.Cu") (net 11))
 (segment (start 134.1 75) (end 135 75) (width 0.3) (layer "F.Cu") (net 11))
 (segment (start 130.366667 75.5) (end 133.6 75.5) (width 0.3) (layer "F.Cu") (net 11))
 (segment (start 137 75) (end 137.2032 74.7968) (width 0.2) (layer "F.Cu") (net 11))
 (segment (start 137.2032 74.7968) (end 138.7 74.7968) (width 0.2) (layer "F.Cu") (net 11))
 (via (at 137 75) (size 0.6) (drill 0.3) (layers "F.Cu" "B.Cu") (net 11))
 (via (at 135 75) (size 0.6) (drill 0.3) (layers "F.Cu" "B.Cu") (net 11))
 (segment (start 135 75) (end 137 75) (width 0.3) (layer "B.Cu") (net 11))
 (segment (start 42.7 77) (end 42.7 76.1) (width 0.3) (layer "F.Cu") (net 4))
 (segment (start 135.5 75.5) (end 135.5 77.05) (width 0.3) (layer "F.Cu") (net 4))
 (segment (start 41.8032 75.2032) (end 42.5 75.9) (width 0.2) (layer "F.Cu") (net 4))
 (segment (start 42.7 76.1) (end 42.5 75.9) (width 0.3) (layer "F.Cu") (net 4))
 (segment (start 135.1 78.35) (end 44.05 78.35) (width 0.3) (layer "F.Cu") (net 4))
 (segment (start 135.7968 75.2032) (end 136.3 75.2032) (width 0.25) (layer "F.Cu") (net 4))
 (segment (start 135.5968 75.4032) (end 135.5 75.5) (width 0.3) (layer "F.Cu") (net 4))
 (segment (start 41.3 75.2032) (end 41.8032 75.2032) (width 0.2) (layer "F.Cu") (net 4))
 (segment (start 135.5968 75.4032) (end 135.7968 75.2032) (width 0.25) (layer "F.Cu") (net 4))
 (segment (start 135.3 78.15) (end 135.1 78.35) (width 0.3) (layer "F.Cu") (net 4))
 (segment (start 44.05 78.35) (end 42.7 77) (width 0.3) (layer "F.Cu") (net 4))
 (via (at 135.5 77.05) (size 0.6) (drill 0.3) (layers "F.Cu" "B.Cu") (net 4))
 (via (at 135.3 78.15) (size 0.6) (drill 0.3) (layers "F.Cu" "B.Cu") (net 4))
 (segment (start 135.5 77.95) (end 135.3 78.15) (width 0.2) (layer "B.Cu") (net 4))
 (segment (start 135.5 77.05) (end 135.5 77.95) (width 0.2) (layer "B.Cu") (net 4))
 (segment (start 44.858062 77.6) (end 137 77.6) (width 0.3) (layer "F.Cu") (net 6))
 (segment (start 138.2968 75.2032) (end 138.3634 75.2032) (width 0.3) (layer "F.Cu") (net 6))
 (segment (start 44.3 75.7) (end 44.3 77.041938) (width 0.3) (layer "F.Cu") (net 6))
 (segment (start 137.6 75.9) (end 138.2968 75.2032) (width 0.3) (layer "F.Cu") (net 6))
 (segment (start 44.3 75.4166) (end 44.0866 75.2032) (width 0.2) (layer "F.Cu") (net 6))
 (segment (start 137 77.6) (end 137.6 77) (width 0.3) (layer "F.Cu") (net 6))
 (segment (start 44.3 77.041938) (end 44.858062 77.6) (width 0.3) (layer "F.Cu") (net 6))
 (segment (start 44.0866 75.2032) (end 43.7 75.2032) (width 0.2) (layer "F.Cu") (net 6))
 (segment (start 138.3634 75.2032) (end 138.7 75.2032) (width 0.2) (layer "F.Cu") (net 6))
 (segment (start 137.6 77) (end 137.6 75.9) (width 0.3) (layer "F.Cu") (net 6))
 (segment (start 44.3 75.7) (end 44.3 75.4166) (width 0.2) (layer "F.Cu") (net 6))
 (segment (start 41.9032 74.7968) (end 41.3 74.7968) (width 0.2) (layer "F.Cu") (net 3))
 (segment (start 136.3 74.7968) (end 135.7968 74.7968) (width 0.2) (layer "F.Cu") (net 3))
 (segment (start 42.4 74) (end 42.4 74.3) (width 0.3) (layer "F.Cu") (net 3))
 (segment (start 135.7968 74.7968) (end 135.4 74.4) (width 0.2) (layer "F.Cu") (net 3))
 (segment (start 135.4 72.8) (end 135.1 72.5) (width 0.3) (layer "F.Cu") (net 3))
 (segment (start 134.4 71.8) (end 44.6 71.8) (width 0.3) (layer "F.Cu") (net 3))
 (segment (start 135.4 74.4) (end 135.4 72.8) (width 0.3) (layer "F.Cu") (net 3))
 (segment (start 42.4 74.3) (end 41.9032 74.7968) (width 0.2) (layer "F.Cu") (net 3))
 (segment (start 44.6 71.8) (end 42.4 74) (width 0.3) (layer "F.Cu") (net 3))
 (segment (start 135.1 72.5) (end 134.4 71.8) (width 0.3) (layer "F.Cu") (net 3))
 (segment (start 51.033333 73.6) (end 50.783333 73.35) (width 0.4) (layer "F.Cu") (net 13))
 (segment (start 52.875 73.6) (end 51.033333 73.6) (width 0.4) (layer "F.Cu") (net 13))
 (segment (start 114.15 76.65) (end 115.9 74.9) (width 0.3) (layer "F.Cu") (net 7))
 (segment (start 115.9 74.9) (end 132.566667 74.9) (width 0.3) (layer "F.Cu") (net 7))
 (segment (start 132.566667 74.9) (end 134.116667 73.35) (width 0.3) (layer "F.Cu") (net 7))
 (segment (start 112.55 76.65) (end 114.15 76.65) (width 0.3) (layer "F.Cu") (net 7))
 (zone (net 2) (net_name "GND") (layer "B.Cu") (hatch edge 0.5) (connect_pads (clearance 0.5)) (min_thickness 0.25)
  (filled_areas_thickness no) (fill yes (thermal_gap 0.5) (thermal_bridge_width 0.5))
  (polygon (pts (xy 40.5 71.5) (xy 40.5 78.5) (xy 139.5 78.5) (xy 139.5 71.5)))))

